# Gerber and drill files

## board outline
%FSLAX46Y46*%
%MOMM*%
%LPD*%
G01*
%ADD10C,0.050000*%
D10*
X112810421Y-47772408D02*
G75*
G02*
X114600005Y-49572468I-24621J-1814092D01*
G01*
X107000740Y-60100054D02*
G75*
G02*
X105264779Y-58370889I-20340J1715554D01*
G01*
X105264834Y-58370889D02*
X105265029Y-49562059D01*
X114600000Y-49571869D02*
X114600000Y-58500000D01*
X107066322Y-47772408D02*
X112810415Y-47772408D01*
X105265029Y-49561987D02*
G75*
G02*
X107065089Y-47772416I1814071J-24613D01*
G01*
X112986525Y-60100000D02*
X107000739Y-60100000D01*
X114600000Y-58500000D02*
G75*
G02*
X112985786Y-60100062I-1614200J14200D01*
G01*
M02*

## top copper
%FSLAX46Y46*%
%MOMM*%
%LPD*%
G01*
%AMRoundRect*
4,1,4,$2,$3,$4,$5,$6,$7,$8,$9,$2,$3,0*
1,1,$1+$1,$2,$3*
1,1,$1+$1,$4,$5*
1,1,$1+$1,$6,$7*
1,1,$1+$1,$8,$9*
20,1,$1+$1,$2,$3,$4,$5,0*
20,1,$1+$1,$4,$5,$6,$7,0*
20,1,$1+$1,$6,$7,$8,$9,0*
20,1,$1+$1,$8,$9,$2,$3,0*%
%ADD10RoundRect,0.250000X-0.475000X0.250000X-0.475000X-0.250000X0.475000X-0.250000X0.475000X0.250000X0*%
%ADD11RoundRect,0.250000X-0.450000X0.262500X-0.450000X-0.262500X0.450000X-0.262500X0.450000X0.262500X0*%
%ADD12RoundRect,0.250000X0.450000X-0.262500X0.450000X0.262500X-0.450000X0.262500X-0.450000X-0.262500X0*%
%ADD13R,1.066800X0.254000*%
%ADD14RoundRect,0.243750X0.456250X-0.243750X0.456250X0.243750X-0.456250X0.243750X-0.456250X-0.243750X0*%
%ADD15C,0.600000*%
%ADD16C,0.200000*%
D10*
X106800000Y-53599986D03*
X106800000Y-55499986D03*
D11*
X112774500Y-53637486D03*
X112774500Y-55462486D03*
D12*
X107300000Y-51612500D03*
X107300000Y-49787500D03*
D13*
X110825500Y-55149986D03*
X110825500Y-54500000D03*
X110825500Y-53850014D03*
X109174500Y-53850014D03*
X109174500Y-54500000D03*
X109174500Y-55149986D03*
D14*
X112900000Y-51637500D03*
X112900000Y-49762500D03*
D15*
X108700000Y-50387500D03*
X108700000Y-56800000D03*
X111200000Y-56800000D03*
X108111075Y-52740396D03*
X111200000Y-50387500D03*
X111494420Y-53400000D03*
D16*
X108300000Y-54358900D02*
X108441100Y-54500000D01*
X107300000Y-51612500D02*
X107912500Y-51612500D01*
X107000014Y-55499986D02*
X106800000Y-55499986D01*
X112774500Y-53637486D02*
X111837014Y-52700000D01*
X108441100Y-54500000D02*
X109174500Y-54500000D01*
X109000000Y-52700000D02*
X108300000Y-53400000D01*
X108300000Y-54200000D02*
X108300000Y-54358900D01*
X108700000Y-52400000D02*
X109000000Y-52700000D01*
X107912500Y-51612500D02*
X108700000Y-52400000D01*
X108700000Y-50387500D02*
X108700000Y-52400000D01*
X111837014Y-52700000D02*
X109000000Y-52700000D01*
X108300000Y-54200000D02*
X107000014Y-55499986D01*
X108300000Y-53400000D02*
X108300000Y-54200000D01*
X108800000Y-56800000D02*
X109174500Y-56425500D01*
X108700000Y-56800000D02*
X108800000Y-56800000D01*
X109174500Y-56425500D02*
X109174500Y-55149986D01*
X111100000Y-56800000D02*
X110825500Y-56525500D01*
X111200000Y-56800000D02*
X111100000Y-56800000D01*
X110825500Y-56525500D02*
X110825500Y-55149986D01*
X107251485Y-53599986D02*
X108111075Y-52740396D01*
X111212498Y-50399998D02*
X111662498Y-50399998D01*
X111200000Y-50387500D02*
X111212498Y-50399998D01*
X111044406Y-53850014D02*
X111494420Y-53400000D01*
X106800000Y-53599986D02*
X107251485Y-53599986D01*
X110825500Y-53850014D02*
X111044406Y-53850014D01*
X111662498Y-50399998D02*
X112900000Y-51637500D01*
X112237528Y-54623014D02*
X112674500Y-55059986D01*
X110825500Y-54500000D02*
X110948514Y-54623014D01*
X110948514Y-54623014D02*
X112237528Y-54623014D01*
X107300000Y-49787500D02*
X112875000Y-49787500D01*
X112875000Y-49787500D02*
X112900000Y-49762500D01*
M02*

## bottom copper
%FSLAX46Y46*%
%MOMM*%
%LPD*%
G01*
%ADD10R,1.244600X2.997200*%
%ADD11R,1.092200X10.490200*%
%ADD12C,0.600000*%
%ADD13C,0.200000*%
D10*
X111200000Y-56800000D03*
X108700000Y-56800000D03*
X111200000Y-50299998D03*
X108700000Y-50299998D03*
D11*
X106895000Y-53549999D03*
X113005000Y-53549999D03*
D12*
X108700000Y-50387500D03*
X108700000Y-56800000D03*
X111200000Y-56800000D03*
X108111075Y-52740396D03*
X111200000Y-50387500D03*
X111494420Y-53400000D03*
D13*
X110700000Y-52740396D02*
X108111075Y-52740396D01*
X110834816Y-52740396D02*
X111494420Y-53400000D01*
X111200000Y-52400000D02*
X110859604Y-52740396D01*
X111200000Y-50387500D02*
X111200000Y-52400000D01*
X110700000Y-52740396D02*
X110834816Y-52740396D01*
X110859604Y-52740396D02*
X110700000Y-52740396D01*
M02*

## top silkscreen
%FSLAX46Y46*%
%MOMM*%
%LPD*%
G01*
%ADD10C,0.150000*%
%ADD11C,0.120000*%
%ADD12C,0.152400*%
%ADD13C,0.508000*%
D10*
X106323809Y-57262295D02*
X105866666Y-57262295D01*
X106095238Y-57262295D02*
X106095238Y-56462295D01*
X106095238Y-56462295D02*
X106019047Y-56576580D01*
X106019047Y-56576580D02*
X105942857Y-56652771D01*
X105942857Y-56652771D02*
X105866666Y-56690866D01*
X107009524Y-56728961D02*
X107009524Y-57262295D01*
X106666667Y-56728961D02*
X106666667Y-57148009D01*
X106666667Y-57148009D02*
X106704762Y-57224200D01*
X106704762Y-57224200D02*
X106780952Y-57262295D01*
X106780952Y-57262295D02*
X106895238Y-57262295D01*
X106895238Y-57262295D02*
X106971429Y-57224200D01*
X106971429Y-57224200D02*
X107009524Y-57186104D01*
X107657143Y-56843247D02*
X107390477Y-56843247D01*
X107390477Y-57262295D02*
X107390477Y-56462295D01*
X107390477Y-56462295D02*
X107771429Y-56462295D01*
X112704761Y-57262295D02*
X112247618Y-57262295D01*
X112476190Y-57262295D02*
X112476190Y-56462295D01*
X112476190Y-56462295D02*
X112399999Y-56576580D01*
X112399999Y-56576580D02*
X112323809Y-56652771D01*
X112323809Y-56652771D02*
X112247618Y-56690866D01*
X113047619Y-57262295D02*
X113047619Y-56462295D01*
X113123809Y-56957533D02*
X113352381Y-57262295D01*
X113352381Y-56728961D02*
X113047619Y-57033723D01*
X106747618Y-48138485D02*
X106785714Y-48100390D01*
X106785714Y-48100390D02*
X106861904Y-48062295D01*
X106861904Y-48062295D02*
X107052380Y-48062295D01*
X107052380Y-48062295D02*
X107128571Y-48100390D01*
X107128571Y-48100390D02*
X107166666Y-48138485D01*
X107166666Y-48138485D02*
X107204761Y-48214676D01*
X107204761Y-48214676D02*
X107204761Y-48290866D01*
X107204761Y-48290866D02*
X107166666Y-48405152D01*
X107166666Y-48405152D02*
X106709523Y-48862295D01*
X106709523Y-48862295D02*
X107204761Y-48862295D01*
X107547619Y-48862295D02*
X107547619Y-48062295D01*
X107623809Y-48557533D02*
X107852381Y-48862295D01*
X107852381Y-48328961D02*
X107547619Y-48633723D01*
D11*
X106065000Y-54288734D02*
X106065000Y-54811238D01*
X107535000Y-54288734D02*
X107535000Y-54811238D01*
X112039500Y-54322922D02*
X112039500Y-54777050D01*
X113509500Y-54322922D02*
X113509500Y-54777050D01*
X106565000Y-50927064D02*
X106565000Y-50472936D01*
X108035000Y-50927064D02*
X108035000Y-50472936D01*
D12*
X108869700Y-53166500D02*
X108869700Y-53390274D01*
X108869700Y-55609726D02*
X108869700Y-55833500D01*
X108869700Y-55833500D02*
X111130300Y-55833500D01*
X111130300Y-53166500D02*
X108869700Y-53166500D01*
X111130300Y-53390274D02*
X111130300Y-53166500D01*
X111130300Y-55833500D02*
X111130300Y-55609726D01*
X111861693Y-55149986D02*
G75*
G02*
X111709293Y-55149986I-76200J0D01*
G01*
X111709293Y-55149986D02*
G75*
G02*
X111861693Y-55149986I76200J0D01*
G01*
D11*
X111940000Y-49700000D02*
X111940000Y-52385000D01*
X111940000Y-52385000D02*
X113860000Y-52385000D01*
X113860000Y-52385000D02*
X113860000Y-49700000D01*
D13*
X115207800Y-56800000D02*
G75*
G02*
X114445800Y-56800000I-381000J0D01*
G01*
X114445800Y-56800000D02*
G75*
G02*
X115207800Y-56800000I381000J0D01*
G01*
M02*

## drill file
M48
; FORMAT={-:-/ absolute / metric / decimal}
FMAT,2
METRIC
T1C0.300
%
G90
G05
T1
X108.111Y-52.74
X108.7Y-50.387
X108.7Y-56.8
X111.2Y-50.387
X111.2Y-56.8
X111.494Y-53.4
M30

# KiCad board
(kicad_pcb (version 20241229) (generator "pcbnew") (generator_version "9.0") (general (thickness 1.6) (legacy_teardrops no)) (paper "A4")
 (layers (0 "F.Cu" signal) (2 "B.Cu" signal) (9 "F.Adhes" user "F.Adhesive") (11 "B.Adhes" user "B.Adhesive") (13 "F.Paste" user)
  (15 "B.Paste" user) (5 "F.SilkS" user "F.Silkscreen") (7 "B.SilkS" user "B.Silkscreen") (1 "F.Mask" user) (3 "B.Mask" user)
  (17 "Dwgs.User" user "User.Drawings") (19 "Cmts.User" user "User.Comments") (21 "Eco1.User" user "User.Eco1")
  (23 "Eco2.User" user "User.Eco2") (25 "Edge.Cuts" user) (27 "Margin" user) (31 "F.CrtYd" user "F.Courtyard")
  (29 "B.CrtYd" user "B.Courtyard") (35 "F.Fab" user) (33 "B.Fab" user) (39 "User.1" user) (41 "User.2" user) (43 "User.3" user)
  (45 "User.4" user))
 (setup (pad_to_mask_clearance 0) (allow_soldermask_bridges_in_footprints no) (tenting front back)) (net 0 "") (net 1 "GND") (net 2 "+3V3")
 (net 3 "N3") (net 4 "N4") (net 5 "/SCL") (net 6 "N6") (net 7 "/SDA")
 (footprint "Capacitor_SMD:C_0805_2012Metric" (layer "F.Cu") (at 106.8 54.549986 -90)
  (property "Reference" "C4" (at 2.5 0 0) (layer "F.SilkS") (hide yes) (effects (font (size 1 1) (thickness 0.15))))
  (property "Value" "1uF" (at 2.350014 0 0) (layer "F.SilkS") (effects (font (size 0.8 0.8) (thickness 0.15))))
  (fp_line (start -0.261252 0.735) (end 0.261252 0.735) (stroke (width 0.12) (type solid)) (layer "F.SilkS"))
  (fp_line (start -0.261252 -0.735) (end 0.261252 -0.735) (stroke (width 0.12) (type solid)) (layer "F.SilkS"))
  (pad "1" smd roundrect (at -0.95 0 270) (size 1 1.45) (layers "F.Cu" "F.Mask" "F.Paste") (roundrect_rratio 0.25) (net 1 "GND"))
  (pad "2" smd roundrect (at 0.95 0 270) (size 1 1.45) (layers "F.Cu" "F.Mask" "F.Paste") (roundrect_rratio 0.25) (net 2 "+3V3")))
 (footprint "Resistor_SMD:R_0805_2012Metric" (layer "F.Cu") (at 112.7745 54.549986 -90)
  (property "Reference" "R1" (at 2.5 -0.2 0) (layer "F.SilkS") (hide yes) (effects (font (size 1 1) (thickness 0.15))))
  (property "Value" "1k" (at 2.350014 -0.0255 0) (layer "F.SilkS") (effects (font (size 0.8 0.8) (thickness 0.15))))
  (fp_line (start -0.227064 0.735) (end 0.227064 0.735) (stroke (width 0.12) (type solid)) (layer "F.SilkS"))
  (fp_line (start -0.227064 -0.735) (end 0.227064 -0.735) (stroke (width 0.12) (type solid)) (layer "F.SilkS"))
  (pad "1" smd roundrect (at -0.9125 0 270) (size 1.025 1.4) (layers "F.Cu" "F.Mask" "F.Paste") (roundrect_rratio 0.243902) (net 2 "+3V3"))
  (pad "2" smd roundrect (at 0.9125 0 270) (size 1.025 1.4) (layers "F.Cu" "F.Mask" "F.Paste") (roundrect_rratio 0.243902) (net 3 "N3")))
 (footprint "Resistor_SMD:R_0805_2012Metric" (layer "F.Cu") (at 107.3 50.7 90)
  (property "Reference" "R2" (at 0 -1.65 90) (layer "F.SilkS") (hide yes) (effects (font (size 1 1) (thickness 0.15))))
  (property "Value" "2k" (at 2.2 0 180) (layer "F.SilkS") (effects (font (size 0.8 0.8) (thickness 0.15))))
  (fp_line (start -0.227064 -0.735) (end 0.227064 -0.735) (stroke (width 0.12) (type solid)) (layer "F.SilkS"))
  (fp_line (start -0.227064 0.735) (end 0.227064 0.735) (stroke (width 0.12) (type solid)) (layer "F.SilkS"))
  (pad "1" smd roundrect (at -0.9125 0 90) (size 1.025 1.4) (layers "F.Cu" "F.Mask" "F.Paste") (roundrect_rratio 0.243902) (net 2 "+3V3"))
  (pad "2" smd roundrect (at 0.9125 0 90) (size 1.025 1.4) (layers "F.Cu" "F.Mask" "F.Paste") (roundrect_rratio 0.243902) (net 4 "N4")))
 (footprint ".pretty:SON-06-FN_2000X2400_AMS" (layer "F.Cu") (at 110 54.5 180)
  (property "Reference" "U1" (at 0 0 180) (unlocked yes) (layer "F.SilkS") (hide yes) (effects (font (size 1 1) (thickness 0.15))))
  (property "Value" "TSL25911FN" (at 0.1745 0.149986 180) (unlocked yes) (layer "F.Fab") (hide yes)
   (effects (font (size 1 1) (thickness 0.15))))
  (fp_line (start 1.1303 1.3335) (end 1.1303 1.109726) (stroke (width 0.1524) (type solid)) (layer "F.SilkS"))
  (fp_line (start 1.1303 -1.109726) (end 1.1303 -1.3335) (stroke (width 0.1524) (type solid)) (layer "F.SilkS"))
  (fp_line (start 1.1303 -1.3335) (end -1.1303 -1.3335) (stroke (width 0.1524) (type solid)) (layer "F.SilkS"))
  (fp_line (start -1.1303 1.3335) (end 1.1303 1.3335) (stroke (width 0.1524) (type solid)) (layer "F.SilkS"))
  (fp_line (start -1.1303 1.109726) (end -1.1303 1.3335) (stroke (width 0.1524) (type solid)) (layer "F.SilkS"))
  (fp_line (start -1.1303 -1.3335) (end -1.1303 -1.109726) (stroke (width 0.1524) (type solid)) (layer "F.SilkS"))
  (fp_circle (center -1.785493 -0.649986) (end -1.709293 -0.649986) (stroke (width 0.1524) (type solid)) (fill no) (layer "F.SilkS"))
  (pad "1" smd rect (at -0.8255 -0.649986 180) (size 1.0668 0.254) (layers "F.Cu" "F.Mask" "F.Paste") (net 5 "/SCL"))
  (pad "2" smd rect (at -0.8255 0 180) (size 1.0668 0.254) (layers "F.Cu" "F.Mask" "F.Paste") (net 3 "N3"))
  (pad "3" smd rect (at -0.8255 0.649986 180) (size 1.0668 0.254) (layers "F.Cu" "F.Mask" "F.Paste") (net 1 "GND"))
  (pad "4" smd rect (at 0.8255 0.649986 180) (size 1.0668 0.254) (layers "F.Cu" "F.Mask" "F.Paste") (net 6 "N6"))
  (pad "5" smd rect (at 0.8255 0 180) (size 1.0668 0.254) (layers "F.Cu" "F.Mask" "F.Paste") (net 2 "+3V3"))
  (pad "6" smd rect (at 0.8255 -0.649986 180) (size 1.0668 0.254) (layers "F.Cu" "F.Mask" "F.Paste") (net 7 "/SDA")))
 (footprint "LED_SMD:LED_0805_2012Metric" (layer "F.Cu") (at 112.9 50.7 90)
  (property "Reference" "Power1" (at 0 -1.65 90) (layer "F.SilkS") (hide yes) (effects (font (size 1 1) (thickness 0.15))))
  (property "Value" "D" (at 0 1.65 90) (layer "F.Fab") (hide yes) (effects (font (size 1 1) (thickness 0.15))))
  (fp_line (start 1 -0.96) (end -1.685 -0.96) (stroke (width 0.12) (type solid)) (layer "F.SilkS"))
  (fp_line (start -1.685 -0.96) (end -1.685 0.96) (stroke (width 0.12) (type solid)) (layer "F.SilkS"))
  (fp_line (start -1.685 0.96) (end 1 0.96) (stroke (width 0.12) (type solid)) (layer "F.SilkS"))
  (pad "1" smd roundrect (at -0.9375 0 90) (size 0.975 1.4) (layers "F.Cu" "F.Mask" "F.Paste") (roundrect_rratio 0.25) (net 1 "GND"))
  (pad "2" smd roundrect (at 0.9375 0 90) (size 0.975 1.4) (layers "F.Cu" "F.Mask" "F.Paste") (roundrect_rratio 0.25) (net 4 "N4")))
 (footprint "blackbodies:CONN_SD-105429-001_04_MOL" (layer "B.Cu") (at 109.95 53.549999)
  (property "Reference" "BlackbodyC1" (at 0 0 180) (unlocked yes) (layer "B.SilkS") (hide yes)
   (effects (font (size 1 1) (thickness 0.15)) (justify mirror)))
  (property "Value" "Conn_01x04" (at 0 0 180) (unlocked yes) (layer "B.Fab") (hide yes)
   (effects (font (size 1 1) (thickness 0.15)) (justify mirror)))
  (fp_circle (center 4.8768 3.250001) (end 5.2578 3.250001) (stroke (width 0.508) (type solid)) (fill no) (layer "F.SilkS"))
  (pad "1" smd rect (at 1.25 3.250001) (size 1.2446 2.9972) (layers "B.Cu" "B.Mask" "B.Paste") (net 5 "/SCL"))
  (pad "2" smd rect (at -1.25 3.250001) (size 1.2446 2.9972) (layers "B.Cu" "B.Mask" "B.Paste") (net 7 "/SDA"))
  (pad "3" smd rect (at 1.25 -3.250001) (size 1.2446 2.9972) (layers "B.Cu" "B.Mask" "B.Paste") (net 1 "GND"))
  (pad "4" smd rect (at -1.25 -3.250001) (size 1.2446 2.9972) (layers "B.Cu" "B.Mask" "B.Paste") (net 2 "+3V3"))
  (pad "5" smd rect (at -3.055 0) (size 1.0922 10.4902) (layers "B.Cu" "B.Mask" "B.Paste"))
  (pad "6" smd rect (at 3.055 0) (size 1.0922 10.4902) (layers "B.Cu" "B.Mask" "B.Paste")))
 (gr_arc (start 112.810421 47.772408) (mid 114.072408 48.307379) (end 114.6 49.572468) (stroke (width 0.05) (type default))
  (layer "Edge.Cuts"))
 (gr_arc (start 107.00074 60.100054) (mid 105.76965 59.600024) (end 105.264834 58.370889) (stroke (width 0.05) (type default))
  (layer "Edge.Cuts"))
 (gr_line (start 105.264834 58.370889) (end 105.265029 49.562059) (stroke (width 0.05) (type default)) (layer "Edge.Cuts"))
 (gr_line (start 114.6 49.571869) (end 114.6 58.5) (stroke (width 0.05) (type default)) (layer "Edge.Cuts"))
 (gr_line (start 107.066322 47.772408) (end 112.810415 47.772408) (stroke (width 0.05) (type default)) (layer "Edge.Cuts"))
 (gr_arc (start 105.265029 49.561987) (mid 105.8 48.3) (end 107.065089 47.772408) (stroke (width 0.05) (type default)) (layer "Edge.Cuts"))
 (gr_line (start 112.986525 60.1) (end 107.000739 60.1) (stroke (width 0.05) (type default)) (layer "Edge.Cuts"))
 (gr_arc (start 114.6 58.5) (mid 114.122215 59.632266) (end 112.985786 60.100063) (stroke (width 0.05) (type default)) (layer "Edge.Cuts"))
 (segment (start 108.3 54.3589) (end 108.4411 54.5) (width 0.2) (layer "F.Cu") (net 2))
 (segment (start 107.3 51.6125) (end 107.9125 51.6125) (width 0.2) (layer "F.Cu") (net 2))
 (segment (start 107.000014 55.499986) (end 106.8 55.499986) (width 0.2) (layer "F.Cu") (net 2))
 (segment (start 112.7745 53.637486) (end 111.837014 52.7) (width 0.2) (layer "F.Cu") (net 2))
 (segment (start 108.4411 54.5) (end 109.1745 54.5) (width 0.2) (layer "F.Cu") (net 2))
 (segment (start 109 52.7) (end 108.3 53.4) (width 0.2) (layer "F.Cu") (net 2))
 (segment (start 108.3 54.2) (end 108.3 54.3589) (width 0.2) (layer "F.Cu") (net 2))
 (segment (start 108.7 52.4) (end 109 52.7) (width 0.2) (layer "F.Cu") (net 2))
 (segment (start 107.9125 51.6125) (end 108.7 52.4) (width 0.2) (layer "F.Cu") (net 2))
 (segment (start 108.7 50.3875) (end 108.7 52.4) (width 0.2) (layer "F.Cu") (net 2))
 (segment (start 111.837014 52.7) (end 109 52.7) (width 0.2) (layer "F.Cu") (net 2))
 (segment (start 108.3 54.2) (end 107.000014 55.499986) (width 0.2) (layer "F.Cu") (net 2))
 (segment (start 108.3 53.4) (end 108.3 54.2) (width 0.2) (layer "F.Cu") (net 2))
 (via (at 108.7 50.3875) (size 0.6) (drill 0.3) (layers "F.Cu" "B.Cu") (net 2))
 (segment (start 108.8 56.8) (end 109.1745 56.4255) (width 0.2) (layer "F.Cu") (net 7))
 (segment (start 108.7 56.8) (end 108.8 56.8) (width 0.2) (layer "F.Cu") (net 7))
 (segment (start 109.1745 56.4255) (end 109.1745 55.149986) (width 0.2) (layer "F.Cu") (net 7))
 (via (at 108.7 56.8) (size 0.6) (drill 0.3) (layers "F.Cu" "B.Cu") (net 7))
 (segment (start 111.1 56.8) (end 110.8255 56.5255) (width 0.2) (layer "F.Cu") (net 5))
 (segment (start 111.2 56.8) (end 111.1 56.8) (width 0.2) (layer "F.Cu") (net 5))
 (segment (start 110.8255 56.5255) (end 110.8255 55.149986) (width 0.2) (layer "F.Cu") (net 5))
 (via (at 111.2 56.8) (size 0.6) (drill 0.3) (layers "F.Cu" "B.Cu") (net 5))
 (segment (start 107.251485 53.599986) (end 108.111075 52.740396) (width 0.2) (layer "F.Cu") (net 1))
 (segment (start 111.212498 50.399998) (end 111.662498 50.399998) (width 0.2) (layer "F.Cu") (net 1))
 (segment (start 111.2 50.3875) (end 111.212498 50.399998) (width 0.2) (layer "F.Cu") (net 1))
 (segment (start 111.044406 53.850014) (end 111.49442 53.4) (width 0.2) (layer "F.Cu") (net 1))
 (segment (start 106.8 53.599986) (end 107.251485 53.599986) (width 0.2) (layer "F.Cu") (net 1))
 (segment (start 110.8255 53.850014) (end 111.044406 53.850014) (width 0.2) (layer "F.Cu") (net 1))
 (segment (start 111.662498 50.399998) (end 112.9 51.6375) (width 0.2) (layer "F.Cu") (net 1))
 (via (at 108.111075 52.740396) (size 0.6) (drill 0.3) (layers "F.Cu" "B.Cu") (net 1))
 (via (at 111.2 50.3875) (size 0.6) (drill 0.3) (layers "F.Cu" "B.Cu") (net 1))
 (via (at 111.49442 53.4) (size 0.6) (drill 0.3) (layers "F.Cu" "B.Cu") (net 1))
 (segment (start 110.7 52.740396) (end 108.111075 52.740396) (width 0.2) (layer "B.Cu") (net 1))
 (segment (start 110.834816 52.740396) (end 111.49442 53.4) (width 0.2) (layer "B.Cu") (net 1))
 (segment (start 111.2 52.4) (end 110.859604 52.740396) (width 0.2) (layer "B.Cu") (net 1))
 (segment (start 111.2 50.3875) (end 111.2 52.4) (width 0.2) (layer "B.Cu") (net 1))
 (segment (start 110.7 52.740396) (end 110.834816 52.740396) (width 0.2) (layer "B.Cu") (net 1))
 (segment (start 110.859604 52.740396) (end 110.7 52.740396) (width 0.2) (layer "B.Cu") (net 1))
 (segment (start 112.237528 54.623014) (end 112.6745 55.059986) (width 0.2) (layer "F.Cu") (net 3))
 (segment (start 110.8255 54.5) (end 110.948514 54.623014) (width 0.2) (layer "F.Cu") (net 3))
 (segment (start 110.948514 54.623014) (end 112.237528 54.623014) (width 0.2) (layer "F.Cu") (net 3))
 (segment (start 107.3 49.7875) (end 112.875 49.7875) (width 0.2) (layer "F.Cu") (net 4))
 (segment (start 112.875 49.7875) (end 112.9 49.7625) (width 0.2) (layer "F.Cu") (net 4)))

